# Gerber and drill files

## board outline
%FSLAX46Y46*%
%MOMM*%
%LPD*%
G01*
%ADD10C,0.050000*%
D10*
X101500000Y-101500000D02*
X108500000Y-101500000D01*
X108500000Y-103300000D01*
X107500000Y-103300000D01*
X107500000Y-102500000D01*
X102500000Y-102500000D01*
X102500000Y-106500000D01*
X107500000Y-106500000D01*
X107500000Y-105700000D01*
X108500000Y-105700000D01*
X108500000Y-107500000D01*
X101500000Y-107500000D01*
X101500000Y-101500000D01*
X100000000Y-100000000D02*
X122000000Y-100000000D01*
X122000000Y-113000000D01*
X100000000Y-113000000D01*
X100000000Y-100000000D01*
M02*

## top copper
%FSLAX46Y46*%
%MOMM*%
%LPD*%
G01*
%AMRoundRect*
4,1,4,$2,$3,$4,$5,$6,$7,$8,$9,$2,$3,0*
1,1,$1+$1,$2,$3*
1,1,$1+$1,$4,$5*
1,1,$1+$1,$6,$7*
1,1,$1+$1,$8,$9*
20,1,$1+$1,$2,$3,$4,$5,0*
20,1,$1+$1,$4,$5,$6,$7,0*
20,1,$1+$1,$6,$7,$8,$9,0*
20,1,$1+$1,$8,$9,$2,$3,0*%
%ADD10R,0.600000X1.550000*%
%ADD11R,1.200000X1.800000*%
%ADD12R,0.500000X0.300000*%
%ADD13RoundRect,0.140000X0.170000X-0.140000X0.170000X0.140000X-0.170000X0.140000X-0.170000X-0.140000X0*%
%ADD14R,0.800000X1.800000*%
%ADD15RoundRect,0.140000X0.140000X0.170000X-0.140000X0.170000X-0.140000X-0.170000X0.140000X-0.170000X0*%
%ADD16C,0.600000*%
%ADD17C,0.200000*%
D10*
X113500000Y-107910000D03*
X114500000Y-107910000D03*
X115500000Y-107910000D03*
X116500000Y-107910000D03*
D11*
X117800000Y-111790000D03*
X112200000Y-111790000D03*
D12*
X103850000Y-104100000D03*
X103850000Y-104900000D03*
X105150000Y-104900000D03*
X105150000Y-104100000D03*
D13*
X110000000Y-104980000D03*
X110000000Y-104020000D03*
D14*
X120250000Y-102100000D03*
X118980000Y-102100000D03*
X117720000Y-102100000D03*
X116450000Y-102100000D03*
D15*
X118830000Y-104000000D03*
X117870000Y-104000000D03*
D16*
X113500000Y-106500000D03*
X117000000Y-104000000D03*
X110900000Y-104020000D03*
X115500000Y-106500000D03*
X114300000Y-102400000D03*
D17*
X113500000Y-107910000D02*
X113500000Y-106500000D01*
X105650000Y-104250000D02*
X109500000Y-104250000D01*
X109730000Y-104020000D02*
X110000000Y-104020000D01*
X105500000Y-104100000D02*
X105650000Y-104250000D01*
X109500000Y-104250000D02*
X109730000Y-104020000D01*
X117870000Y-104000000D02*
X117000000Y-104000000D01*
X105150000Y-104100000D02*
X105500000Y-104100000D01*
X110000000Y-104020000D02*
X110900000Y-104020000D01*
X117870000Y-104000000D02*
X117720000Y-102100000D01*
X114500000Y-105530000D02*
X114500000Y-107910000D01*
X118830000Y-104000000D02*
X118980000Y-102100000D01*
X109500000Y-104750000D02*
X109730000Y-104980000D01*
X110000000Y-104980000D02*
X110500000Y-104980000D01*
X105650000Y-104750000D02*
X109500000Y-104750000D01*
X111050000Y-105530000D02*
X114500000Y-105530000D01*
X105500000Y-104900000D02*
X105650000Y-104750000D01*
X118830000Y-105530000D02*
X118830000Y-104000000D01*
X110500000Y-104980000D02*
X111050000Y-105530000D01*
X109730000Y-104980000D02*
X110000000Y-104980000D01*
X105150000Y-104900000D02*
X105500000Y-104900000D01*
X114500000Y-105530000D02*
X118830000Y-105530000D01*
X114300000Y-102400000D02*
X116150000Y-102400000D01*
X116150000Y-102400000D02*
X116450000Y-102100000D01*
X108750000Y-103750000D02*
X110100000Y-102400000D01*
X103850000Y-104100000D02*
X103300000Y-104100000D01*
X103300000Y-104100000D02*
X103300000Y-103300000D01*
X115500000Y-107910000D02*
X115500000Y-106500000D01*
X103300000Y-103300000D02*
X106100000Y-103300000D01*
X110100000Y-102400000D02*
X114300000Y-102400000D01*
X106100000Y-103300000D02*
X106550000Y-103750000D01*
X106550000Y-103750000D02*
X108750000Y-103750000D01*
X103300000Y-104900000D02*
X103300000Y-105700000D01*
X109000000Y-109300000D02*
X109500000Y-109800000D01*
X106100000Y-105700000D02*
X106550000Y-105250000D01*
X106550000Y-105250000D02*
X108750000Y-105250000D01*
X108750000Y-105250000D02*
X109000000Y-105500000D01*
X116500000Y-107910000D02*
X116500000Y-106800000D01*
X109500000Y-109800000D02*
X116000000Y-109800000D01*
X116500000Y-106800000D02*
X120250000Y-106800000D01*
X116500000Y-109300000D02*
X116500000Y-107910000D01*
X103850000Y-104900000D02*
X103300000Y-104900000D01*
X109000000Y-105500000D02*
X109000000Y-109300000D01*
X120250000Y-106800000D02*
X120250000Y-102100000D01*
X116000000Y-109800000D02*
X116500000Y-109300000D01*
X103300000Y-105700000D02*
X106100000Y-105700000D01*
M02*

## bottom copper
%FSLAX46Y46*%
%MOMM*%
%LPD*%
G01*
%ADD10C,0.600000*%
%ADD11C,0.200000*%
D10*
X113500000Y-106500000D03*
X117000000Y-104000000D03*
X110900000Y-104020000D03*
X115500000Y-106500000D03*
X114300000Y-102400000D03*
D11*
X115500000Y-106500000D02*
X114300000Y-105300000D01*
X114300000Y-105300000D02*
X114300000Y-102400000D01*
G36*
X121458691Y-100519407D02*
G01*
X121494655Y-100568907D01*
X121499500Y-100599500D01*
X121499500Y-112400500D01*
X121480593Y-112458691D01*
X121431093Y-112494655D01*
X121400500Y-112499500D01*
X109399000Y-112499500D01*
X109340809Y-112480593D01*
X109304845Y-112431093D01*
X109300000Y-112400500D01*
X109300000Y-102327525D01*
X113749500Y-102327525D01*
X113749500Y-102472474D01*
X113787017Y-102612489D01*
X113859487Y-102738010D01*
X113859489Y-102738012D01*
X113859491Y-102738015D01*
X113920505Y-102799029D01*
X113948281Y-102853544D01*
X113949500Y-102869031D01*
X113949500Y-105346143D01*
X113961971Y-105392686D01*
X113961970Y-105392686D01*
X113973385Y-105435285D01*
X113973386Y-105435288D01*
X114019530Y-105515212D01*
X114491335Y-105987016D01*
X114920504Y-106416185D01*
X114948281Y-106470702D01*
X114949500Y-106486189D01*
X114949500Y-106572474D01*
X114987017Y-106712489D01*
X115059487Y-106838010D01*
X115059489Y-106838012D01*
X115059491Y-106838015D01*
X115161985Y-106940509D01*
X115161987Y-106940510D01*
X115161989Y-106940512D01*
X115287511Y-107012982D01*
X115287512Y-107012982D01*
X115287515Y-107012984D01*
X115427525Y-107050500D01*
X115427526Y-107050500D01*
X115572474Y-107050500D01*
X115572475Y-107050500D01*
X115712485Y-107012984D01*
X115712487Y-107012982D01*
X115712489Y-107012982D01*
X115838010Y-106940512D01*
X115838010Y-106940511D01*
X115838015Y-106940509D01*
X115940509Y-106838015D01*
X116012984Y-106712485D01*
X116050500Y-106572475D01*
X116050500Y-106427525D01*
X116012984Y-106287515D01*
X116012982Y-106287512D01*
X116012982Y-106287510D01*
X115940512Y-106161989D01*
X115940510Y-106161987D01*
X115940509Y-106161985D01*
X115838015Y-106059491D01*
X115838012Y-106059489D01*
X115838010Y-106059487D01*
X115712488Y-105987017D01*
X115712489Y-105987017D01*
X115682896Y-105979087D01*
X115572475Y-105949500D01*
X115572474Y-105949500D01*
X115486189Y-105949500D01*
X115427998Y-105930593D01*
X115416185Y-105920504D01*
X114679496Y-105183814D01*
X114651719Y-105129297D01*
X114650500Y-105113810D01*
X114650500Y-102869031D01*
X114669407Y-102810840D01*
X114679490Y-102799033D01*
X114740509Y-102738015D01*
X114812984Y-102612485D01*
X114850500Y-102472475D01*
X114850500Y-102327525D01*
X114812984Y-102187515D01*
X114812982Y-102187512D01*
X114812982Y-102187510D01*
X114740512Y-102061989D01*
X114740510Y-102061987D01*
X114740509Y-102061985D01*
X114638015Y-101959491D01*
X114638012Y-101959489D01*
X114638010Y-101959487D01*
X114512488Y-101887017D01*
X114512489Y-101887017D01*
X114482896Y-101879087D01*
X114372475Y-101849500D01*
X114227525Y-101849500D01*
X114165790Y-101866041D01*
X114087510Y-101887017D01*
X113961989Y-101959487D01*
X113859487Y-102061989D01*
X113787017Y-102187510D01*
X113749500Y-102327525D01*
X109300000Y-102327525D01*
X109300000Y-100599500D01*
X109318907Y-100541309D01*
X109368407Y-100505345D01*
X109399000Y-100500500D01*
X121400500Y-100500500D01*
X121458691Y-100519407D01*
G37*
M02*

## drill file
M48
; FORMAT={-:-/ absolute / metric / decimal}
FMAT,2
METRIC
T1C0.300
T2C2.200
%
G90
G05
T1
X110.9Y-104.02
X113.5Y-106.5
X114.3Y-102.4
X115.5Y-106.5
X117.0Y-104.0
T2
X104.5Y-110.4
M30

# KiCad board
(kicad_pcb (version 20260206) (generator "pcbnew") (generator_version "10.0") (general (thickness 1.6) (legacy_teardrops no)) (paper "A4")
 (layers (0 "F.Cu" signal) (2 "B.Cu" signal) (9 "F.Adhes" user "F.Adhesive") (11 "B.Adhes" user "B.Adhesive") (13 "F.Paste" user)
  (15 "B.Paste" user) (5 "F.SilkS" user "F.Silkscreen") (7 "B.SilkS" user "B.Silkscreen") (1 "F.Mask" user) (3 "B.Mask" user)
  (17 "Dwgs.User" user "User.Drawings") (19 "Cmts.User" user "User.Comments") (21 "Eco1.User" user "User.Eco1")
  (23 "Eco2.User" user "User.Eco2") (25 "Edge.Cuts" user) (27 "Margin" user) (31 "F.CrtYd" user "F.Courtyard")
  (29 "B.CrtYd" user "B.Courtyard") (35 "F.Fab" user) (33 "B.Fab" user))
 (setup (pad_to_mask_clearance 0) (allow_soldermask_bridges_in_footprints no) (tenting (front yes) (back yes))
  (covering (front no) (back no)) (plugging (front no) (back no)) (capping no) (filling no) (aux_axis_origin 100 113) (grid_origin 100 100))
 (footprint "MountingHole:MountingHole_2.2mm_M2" (layer "F.Cu") (at 104.5 110.4 -90)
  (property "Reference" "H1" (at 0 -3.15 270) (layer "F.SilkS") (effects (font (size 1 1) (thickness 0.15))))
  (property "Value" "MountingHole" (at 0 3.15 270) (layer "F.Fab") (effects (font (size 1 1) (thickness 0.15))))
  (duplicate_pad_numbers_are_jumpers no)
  (pad "" np_thru_hole circle (at 0 0 270) (size 2.2 2.2) (drill 2.2) (layers "*.Cu" "*.Mask")))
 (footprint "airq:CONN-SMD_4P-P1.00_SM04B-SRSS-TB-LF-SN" (layer "F.Cu") (at 115 109.85)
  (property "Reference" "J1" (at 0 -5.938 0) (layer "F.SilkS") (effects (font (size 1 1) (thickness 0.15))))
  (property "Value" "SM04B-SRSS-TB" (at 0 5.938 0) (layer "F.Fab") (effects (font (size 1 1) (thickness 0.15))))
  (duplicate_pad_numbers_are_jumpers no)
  (pad "1" smd rect (at -1.5 -1.94) (size 0.6 1.55) (layers "F.Cu" "F.Mask" "F.Paste") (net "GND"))
  (pad "2" smd rect (at -0.5 -1.94) (size 0.6 1.55) (layers "F.Cu" "F.Mask" "F.Paste") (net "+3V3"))
  (pad "3" smd rect (at 0.5 -1.94) (size 0.6 1.55) (layers "F.Cu" "F.Mask" "F.Paste") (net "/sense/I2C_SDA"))
  (pad "4" smd rect (at 1.5 -1.94) (size 0.6 1.55) (layers "F.Cu" "F.Mask" "F.Paste") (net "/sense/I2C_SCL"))
  (pad "5" smd rect (at 2.8 1.94) (size 1.2 1.8) (layers "F.Cu" "F.Mask" "F.Paste") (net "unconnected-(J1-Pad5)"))
  (pad "6" smd rect (at -2.8 1.94) (size 1.2 1.8) (layers "F.Cu" "F.Mask" "F.Paste") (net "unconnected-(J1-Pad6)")))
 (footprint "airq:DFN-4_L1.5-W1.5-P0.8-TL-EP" (layer "F.Cu") (at 104.5 104.5)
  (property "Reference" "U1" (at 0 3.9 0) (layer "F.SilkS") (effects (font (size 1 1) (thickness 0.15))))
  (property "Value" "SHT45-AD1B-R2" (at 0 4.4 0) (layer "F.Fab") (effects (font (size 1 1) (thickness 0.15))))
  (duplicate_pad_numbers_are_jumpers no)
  (pad "1" smd rect (at -0.65 -0.4) (size 0.5 0.3) (layers "F.Cu" "F.Mask" "F.Paste") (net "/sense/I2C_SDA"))
  (pad "2" smd rect (at -0.65 0.4) (size 0.5 0.3) (layers "F.Cu" "F.Mask" "F.Paste") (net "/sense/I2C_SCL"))
  (pad "3" smd rect (at 0.65 0.4) (size 0.5 0.3) (layers "F.Cu" "F.Mask" "F.Paste") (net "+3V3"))
  (pad "4" smd rect (at 0.65 -0.4) (size 0.5 0.3) (layers "F.Cu" "F.Mask" "F.Paste") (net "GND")))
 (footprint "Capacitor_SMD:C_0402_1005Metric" (layer "F.Cu") (at 110 104.5 90)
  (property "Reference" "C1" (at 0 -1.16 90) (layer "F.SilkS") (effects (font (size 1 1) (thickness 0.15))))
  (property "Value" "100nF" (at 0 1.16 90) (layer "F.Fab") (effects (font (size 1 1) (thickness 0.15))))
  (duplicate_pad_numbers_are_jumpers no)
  (pad "1" smd roundrect (at -0.48 0 90) (size 0.56 0.62) (layers "F.Cu" "F.Mask" "F.Paste") (roundrect_rratio 0.25) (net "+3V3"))
  (pad "2" smd roundrect (at 0.48 0 90) (size 0.56 0.62) (layers "F.Cu" "F.Mask" "F.Paste") (roundrect_rratio 0.25) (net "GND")))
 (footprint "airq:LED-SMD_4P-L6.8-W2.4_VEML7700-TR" (layer "F.Cu") (at 118.35 102.1)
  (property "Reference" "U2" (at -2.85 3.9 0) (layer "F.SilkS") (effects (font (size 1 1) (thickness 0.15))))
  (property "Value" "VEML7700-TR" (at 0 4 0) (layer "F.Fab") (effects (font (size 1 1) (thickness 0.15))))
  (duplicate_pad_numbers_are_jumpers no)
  (pad "1" smd rect (at 1.9 0) (size 0.8 1.8) (layers "F.Cu" "F.Mask" "F.Paste") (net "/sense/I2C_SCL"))
  (pad "2" smd rect (at 0.63 0) (size 0.8 1.8) (layers "F.Cu" "F.Mask" "F.Paste") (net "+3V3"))
  (pad "3" smd rect (at -0.63 0) (size 0.8 1.8) (layers "F.Cu" "F.Mask" "F.Paste") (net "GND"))
  (pad "4" smd rect (at -1.9 0) (size 0.8 1.8) (layers "F.Cu" "F.Mask" "F.Paste") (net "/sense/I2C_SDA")))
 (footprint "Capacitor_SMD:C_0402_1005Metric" (layer "F.Cu") (at 118.35 104 180)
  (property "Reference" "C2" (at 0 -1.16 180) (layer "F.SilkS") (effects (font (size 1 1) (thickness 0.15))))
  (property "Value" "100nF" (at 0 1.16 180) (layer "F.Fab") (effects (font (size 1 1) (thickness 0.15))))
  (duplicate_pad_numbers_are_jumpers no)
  (pad "1" smd roundrect (at -0.48 0 180) (size 0.56 0.62) (layers "F.Cu" "F.Mask" "F.Paste") (roundrect_rratio 0.25) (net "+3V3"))
  (pad "2" smd roundrect (at 0.48 0 180) (size 0.56 0.62) (layers "F.Cu" "F.Mask" "F.Paste") (roundrect_rratio 0.25) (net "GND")))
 (gr_poly
  (pts (xy 101.5 101.5) (xy 108.5 101.5) (xy 108.5 103.3) (xy 107.5 103.3) (xy 107.5 102.5) (xy 102.5 102.5) (xy 102.5 106.5)
   (xy 107.5 106.5) (xy 107.5 105.7) (xy 108.5 105.7) (xy 108.5 107.5) (xy 101.5 107.5))
  (stroke (width 0.05) (type default)) (fill no) (layer "Edge.Cuts"))
 (gr_rect (start 100 100) (end 122 113) (stroke (width 0.05) (type default)) (fill no) (layer "Edge.Cuts"))
 (segment (start 113.5 107.91) (end 113.5 106.5) (width 0.2) (layer "F.Cu") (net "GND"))
 (segment (start 105.65 104.25) (end 109.5 104.25) (width 0.2) (layer "F.Cu") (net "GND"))
 (segment (start 109.73 104.02) (end 110 104.02) (width 0.2) (layer "F.Cu") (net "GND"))
 (segment (start 105.5 104.1) (end 105.65 104.25) (width 0.2) (layer "F.Cu") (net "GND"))
 (segment (start 109.5 104.25) (end 109.73 104.02) (width 0.2) (layer "F.Cu") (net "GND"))
 (segment (start 117.87 104) (end 117 104) (width 0.2) (layer "F.Cu") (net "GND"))
 (segment (start 105.15 104.1) (end 105.5 104.1) (width 0.2) (layer "F.Cu") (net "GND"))
 (segment (start 110 104.02) (end 110.9 104.02) (width 0.2) (layer "F.Cu") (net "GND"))
 (segment (start 117.87 104) (end 117.72 102.1) (width 0.2) (layer "F.Cu") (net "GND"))
 (via (at 113.5 106.5) (size 0.6) (drill 0.3) (layers "F.Cu" "B.Cu") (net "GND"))
 (via (at 117 104) (size 0.6) (drill 0.3) (layers "F.Cu" "B.Cu") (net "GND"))
 (via (at 110.9 104.02) (size 0.6) (drill 0.3) (layers "F.Cu" "B.Cu") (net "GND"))
 (segment (start 114.5 105.53) (end 114.5 107.91) (width 0.2) (layer "F.Cu") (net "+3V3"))
 (segment (start 118.83 104) (end 118.98 102.1) (width 0.2) (layer "F.Cu") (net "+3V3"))
 (segment (start 109.5 104.75) (end 109.73 104.98) (width 0.2) (layer "F.Cu") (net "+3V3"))
 (segment (start 110 104.98) (end 110.5 104.98) (width 0.2) (layer "F.Cu") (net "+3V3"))
 (segment (start 105.65 104.75) (end 109.5 104.75) (width 0.2) (layer "F.Cu") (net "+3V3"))
 (segment (start 111.05 105.53) (end 114.5 105.53) (width 0.2) (layer "F.Cu") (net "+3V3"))
 (segment (start 105.5 104.9) (end 105.65 104.75) (width 0.2) (layer "F.Cu") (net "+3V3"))
 (segment (start 118.83 105.53) (end 118.83 104) (width 0.2) (layer "F.Cu") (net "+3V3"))
 (segment (start 110.5 104.98) (end 111.05 105.53) (width 0.2) (layer "F.Cu") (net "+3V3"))
 (segment (start 109.73 104.98) (end 110 104.98) (width 0.2) (layer "F.Cu") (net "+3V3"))
 (segment (start 105.15 104.9) (end 105.5 104.9) (width 0.2) (layer "F.Cu") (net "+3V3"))
 (segment (start 114.5 105.53) (end 118.83 105.53) (width 0.2) (layer "F.Cu") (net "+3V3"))
 (segment (start 114.3 102.4) (end 116.15 102.4) (width 0.2) (layer "F.Cu") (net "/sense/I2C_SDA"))
 (segment (start 116.15 102.4) (end 116.45 102.1) (width 0.2) (layer "F.Cu") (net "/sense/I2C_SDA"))
 (segment (start 108.75 103.75) (end 110.1 102.4) (width 0.2) (layer "F.Cu") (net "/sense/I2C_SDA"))
 (segment (start 103.85 104.1) (end 103.3 104.1) (width 0.2) (layer "F.Cu") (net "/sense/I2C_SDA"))
 (segment (start 103.3 104.1) (end 103.3 103.3) (width 0.2) (layer "F.Cu") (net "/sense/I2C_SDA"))
 (segment (start 115.5 107.91) (end 115.5 106.5) (width 0.2) (layer "F.Cu") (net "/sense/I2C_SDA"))
 (segment (start 103.3 103.3) (end 106.1 103.3) (width 0.2) (layer "F.Cu") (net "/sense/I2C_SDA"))
 (segment (start 110.1 102.4) (end 114.3 102.4) (width 0.2) (layer "F.Cu") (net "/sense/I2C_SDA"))
 (segment (start 106.1 103.3) (end 106.55 103.75) (width 0.2) (layer "F.Cu") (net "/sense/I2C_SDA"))
 (segment (start 106.55 103.75) (end 108.75 103.75) (width 0.2) (layer "F.Cu") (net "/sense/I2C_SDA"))
 (via (at 115.5 106.5) (size 0.6) (drill 0.3) (layers "F.Cu" "B.Cu") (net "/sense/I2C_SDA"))
 (via (at 114.3 102.4) (size 0.6) (drill 0.3) (layers "F.Cu" "B.Cu") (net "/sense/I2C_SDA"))
 (segment (start 115.5 106.5) (end 114.3 105.3) (width 0.2) (layer "B.Cu") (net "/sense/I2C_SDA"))
 (segment (start 114.3 105.3) (end 114.3 102.4) (width 0.2) (layer "B.Cu") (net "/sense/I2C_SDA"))
 (segment (start 103.3 104.9) (end 103.3 105.7) (width 0.2) (layer "F.Cu") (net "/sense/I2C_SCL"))
 (segment (start 109 109.3) (end 109.5 109.8) (width 0.2) (layer "F.Cu") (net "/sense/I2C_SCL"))
 (segment (start 106.1 105.7) (end 106.55 105.25) (width 0.2) (layer "F.Cu") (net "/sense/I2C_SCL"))
 (segment (start 106.55 105.25) (end 108.75 105.25) (width 0.2) (layer "F.Cu") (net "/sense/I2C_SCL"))
 (segment (start 108.75 105.25) (end 109 105.5) (width 0.2) (layer "F.Cu") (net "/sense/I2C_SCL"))
 (segment (start 116.5 107.91) (end 116.5 106.8) (width 0.2) (layer "F.Cu") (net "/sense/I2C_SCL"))
 (segment (start 109.5 109.8) (end 116 109.8) (width 0.2) (layer "F.Cu") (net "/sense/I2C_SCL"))
 (segment (start 116.5 106.8) (end 120.25 106.8) (width 0.2) (layer "F.Cu") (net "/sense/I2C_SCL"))
 (segment (start 116.5 109.3) (end 116.5 107.91) (width 0.2) (layer "F.Cu") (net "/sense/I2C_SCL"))
 (segment (start 103.85 104.9) (end 103.3 104.9) (width 0.2) (layer "F.Cu") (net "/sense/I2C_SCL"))
 (segment (start 109 105.5) (end 109 109.3) (width 0.2) (layer "F.Cu") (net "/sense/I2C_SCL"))
 (segment (start 120.25 106.8) (end 120.25 102.1) (width 0.2) (layer "F.Cu") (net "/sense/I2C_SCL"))
 (segment (start 116 109.8) (end 116.5 109.3) (width 0.2) (layer "F.Cu") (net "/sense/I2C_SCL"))
 (segment (start 103.3 105.7) (end 106.1 105.7) (width 0.2) (layer "F.Cu") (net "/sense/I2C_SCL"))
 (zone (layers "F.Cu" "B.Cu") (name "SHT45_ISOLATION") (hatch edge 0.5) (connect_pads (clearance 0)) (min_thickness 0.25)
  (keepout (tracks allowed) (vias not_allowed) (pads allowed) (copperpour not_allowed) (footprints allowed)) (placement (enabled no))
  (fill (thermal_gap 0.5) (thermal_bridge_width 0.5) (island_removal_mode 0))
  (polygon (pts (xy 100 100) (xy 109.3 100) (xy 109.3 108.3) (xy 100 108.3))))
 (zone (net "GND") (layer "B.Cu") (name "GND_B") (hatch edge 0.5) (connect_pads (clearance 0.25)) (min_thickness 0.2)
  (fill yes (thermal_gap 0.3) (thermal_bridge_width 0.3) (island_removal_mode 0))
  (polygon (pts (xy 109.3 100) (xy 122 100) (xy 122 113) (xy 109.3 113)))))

